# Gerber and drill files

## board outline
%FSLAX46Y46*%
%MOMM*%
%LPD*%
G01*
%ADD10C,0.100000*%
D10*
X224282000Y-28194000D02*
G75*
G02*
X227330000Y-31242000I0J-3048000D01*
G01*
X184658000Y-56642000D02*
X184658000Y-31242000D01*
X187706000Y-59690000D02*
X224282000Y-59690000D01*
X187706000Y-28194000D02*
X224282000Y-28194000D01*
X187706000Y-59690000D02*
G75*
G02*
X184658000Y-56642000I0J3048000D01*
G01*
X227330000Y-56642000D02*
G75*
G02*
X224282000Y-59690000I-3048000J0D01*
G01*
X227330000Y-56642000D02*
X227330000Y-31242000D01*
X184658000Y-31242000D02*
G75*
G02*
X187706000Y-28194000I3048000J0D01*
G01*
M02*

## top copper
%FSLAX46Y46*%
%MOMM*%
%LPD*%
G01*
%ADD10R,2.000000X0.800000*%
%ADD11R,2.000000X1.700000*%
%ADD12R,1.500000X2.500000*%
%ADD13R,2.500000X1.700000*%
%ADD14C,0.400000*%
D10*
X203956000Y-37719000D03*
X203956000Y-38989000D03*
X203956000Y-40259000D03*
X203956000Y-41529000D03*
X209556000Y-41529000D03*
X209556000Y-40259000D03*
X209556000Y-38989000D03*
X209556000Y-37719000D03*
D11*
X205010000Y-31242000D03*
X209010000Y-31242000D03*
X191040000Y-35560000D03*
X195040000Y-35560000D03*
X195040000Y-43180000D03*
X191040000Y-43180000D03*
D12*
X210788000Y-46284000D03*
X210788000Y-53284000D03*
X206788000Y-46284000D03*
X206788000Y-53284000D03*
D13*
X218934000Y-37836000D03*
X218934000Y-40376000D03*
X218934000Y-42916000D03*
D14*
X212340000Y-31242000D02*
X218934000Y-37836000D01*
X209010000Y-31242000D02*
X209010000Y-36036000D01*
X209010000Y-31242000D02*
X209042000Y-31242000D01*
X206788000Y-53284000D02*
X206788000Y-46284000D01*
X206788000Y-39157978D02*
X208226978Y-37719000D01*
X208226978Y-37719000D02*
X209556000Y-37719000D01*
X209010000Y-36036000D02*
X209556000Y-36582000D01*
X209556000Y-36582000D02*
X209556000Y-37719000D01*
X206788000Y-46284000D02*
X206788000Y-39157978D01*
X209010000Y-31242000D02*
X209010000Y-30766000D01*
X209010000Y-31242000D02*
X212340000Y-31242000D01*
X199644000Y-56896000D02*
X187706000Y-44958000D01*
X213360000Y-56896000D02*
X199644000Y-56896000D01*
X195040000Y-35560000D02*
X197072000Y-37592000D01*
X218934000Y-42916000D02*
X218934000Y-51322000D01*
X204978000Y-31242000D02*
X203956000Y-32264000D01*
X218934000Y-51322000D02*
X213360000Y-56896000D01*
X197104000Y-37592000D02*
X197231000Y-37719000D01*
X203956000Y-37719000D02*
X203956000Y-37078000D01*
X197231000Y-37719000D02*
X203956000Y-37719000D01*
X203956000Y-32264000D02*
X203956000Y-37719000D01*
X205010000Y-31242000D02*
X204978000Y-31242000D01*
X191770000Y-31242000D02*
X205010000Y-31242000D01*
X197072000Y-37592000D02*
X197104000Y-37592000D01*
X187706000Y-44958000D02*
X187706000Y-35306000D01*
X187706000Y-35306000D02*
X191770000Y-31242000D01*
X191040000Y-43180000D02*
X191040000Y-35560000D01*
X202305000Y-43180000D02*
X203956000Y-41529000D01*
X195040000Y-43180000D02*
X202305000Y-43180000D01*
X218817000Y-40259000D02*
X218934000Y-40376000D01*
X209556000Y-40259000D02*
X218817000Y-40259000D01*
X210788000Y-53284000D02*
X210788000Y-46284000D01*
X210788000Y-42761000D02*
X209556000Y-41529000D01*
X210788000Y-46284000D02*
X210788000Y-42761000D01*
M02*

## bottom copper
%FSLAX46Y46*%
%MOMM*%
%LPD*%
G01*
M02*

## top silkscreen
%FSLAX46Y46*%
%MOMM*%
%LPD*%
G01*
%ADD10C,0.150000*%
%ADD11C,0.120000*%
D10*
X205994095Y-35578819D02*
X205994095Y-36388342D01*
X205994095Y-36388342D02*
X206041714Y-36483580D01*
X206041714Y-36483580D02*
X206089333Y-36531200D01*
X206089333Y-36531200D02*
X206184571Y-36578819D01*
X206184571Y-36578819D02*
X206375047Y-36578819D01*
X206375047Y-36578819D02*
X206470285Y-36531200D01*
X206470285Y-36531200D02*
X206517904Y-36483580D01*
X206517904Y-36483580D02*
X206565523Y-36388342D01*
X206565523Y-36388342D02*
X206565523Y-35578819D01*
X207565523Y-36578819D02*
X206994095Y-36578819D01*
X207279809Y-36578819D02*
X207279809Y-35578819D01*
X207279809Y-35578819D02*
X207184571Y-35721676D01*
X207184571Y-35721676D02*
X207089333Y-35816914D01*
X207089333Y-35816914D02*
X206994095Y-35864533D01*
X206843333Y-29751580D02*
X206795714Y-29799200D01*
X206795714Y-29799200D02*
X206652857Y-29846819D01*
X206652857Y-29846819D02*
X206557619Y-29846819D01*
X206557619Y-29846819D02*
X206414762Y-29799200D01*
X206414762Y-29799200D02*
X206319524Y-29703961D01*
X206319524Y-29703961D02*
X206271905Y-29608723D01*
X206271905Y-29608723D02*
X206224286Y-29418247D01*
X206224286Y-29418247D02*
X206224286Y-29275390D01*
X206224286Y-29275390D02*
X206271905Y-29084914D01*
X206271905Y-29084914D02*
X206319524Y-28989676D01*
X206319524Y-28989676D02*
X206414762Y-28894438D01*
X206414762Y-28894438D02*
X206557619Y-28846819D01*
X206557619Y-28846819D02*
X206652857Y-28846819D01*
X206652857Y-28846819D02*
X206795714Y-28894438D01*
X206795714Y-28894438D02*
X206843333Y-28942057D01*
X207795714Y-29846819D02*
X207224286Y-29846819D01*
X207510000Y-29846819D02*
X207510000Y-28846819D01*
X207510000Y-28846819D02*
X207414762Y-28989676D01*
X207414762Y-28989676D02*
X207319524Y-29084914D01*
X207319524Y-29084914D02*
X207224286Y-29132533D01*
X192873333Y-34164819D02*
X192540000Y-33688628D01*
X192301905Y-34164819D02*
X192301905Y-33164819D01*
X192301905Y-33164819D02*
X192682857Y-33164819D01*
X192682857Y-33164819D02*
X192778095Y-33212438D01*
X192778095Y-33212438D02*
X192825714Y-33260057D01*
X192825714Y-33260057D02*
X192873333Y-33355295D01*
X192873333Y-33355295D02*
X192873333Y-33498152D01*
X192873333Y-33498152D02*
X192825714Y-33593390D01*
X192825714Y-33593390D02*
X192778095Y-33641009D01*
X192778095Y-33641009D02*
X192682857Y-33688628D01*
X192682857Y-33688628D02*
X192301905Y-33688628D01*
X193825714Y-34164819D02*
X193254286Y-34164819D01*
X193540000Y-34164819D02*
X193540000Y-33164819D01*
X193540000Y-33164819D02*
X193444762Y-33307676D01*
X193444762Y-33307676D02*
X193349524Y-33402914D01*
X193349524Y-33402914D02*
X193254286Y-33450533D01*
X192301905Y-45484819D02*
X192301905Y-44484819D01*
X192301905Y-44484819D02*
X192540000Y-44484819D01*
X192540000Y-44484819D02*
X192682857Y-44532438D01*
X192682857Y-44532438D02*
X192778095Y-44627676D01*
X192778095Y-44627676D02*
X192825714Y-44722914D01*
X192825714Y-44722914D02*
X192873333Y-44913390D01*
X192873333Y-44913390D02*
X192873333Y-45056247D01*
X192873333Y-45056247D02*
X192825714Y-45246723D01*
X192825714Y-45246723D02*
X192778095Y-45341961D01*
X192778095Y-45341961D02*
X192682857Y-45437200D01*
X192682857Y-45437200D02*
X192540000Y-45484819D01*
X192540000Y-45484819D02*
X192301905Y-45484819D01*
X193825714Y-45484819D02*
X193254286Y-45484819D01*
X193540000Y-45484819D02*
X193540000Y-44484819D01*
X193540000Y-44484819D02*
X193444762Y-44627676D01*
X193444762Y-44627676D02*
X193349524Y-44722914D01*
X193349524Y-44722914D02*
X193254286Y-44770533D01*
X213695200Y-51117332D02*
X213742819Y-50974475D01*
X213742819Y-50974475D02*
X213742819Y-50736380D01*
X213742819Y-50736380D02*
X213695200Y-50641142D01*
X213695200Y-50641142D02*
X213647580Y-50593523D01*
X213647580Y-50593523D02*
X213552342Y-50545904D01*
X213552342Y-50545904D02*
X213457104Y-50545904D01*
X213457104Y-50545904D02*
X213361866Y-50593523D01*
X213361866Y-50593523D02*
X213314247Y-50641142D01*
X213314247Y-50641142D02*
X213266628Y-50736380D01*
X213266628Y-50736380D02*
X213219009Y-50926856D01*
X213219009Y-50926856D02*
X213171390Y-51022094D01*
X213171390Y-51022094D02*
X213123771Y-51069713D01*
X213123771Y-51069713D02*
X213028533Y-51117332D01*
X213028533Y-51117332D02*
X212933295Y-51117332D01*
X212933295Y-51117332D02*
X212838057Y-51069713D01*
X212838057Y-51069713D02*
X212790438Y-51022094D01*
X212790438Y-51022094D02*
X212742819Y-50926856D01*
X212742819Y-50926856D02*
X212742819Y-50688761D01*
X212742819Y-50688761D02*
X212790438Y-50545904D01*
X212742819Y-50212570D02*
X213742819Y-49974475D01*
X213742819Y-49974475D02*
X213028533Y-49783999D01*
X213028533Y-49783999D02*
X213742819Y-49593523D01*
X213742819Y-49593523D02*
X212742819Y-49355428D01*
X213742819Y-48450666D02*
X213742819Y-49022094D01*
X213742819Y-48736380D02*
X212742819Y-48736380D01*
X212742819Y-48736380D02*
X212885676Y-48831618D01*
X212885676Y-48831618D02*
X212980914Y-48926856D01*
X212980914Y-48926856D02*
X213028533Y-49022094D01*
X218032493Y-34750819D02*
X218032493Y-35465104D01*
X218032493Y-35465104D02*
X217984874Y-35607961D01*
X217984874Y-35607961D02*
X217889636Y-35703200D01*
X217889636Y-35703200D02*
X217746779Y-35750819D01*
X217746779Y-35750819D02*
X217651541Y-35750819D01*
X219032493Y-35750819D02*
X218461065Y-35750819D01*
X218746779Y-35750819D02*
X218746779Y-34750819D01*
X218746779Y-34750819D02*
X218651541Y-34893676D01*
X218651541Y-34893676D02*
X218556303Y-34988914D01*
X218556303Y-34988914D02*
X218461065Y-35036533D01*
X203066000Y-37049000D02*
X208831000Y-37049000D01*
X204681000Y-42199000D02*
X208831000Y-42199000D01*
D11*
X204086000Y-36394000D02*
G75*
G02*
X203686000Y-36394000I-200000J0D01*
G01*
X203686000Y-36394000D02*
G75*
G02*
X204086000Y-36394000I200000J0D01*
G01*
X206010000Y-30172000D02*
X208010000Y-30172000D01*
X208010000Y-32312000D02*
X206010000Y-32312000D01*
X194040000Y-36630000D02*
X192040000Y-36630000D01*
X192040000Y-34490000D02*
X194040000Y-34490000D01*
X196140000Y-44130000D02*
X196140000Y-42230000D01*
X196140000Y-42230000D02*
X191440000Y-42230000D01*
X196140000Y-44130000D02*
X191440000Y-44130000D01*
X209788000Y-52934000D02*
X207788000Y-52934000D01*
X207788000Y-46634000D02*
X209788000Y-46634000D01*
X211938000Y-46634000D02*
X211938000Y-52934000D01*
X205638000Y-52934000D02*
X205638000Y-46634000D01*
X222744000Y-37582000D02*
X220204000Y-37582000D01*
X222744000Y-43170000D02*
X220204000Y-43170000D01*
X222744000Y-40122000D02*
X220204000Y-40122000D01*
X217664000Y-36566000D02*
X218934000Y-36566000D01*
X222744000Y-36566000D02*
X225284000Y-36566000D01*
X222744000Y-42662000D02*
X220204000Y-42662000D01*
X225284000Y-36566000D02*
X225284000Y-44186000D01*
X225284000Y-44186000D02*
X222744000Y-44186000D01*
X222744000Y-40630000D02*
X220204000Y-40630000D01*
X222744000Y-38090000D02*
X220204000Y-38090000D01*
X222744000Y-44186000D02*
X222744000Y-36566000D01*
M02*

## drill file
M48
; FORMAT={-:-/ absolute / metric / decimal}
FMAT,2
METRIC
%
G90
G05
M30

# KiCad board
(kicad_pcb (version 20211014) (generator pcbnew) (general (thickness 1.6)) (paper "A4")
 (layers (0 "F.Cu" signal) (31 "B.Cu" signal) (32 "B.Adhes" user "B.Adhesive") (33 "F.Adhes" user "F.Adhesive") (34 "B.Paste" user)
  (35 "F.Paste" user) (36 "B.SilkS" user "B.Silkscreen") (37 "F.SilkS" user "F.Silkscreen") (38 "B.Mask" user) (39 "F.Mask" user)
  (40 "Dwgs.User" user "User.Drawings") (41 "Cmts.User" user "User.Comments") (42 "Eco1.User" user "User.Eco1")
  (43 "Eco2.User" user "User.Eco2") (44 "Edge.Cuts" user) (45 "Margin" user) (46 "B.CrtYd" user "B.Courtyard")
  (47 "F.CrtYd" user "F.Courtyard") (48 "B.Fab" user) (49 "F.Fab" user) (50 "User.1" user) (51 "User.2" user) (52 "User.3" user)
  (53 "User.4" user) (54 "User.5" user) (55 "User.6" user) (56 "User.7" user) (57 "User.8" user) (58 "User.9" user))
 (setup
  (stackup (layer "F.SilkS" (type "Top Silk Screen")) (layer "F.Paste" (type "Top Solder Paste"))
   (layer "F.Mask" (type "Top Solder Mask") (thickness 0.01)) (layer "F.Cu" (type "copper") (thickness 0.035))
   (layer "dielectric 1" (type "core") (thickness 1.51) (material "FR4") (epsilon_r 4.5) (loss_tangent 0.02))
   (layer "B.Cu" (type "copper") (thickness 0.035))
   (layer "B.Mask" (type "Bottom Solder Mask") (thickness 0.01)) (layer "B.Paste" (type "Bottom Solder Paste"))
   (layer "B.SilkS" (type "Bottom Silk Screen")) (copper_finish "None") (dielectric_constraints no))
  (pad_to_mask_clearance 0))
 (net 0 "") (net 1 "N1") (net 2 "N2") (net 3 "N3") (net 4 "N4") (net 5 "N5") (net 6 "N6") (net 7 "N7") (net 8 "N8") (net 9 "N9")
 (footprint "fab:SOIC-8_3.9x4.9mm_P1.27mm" (layer "F.Cu") (at 206.756 39.624)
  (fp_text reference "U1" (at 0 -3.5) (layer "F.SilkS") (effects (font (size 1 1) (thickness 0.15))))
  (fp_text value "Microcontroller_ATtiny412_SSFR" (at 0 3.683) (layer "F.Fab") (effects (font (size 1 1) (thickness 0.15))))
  (fp_line (start -3.69 -2.575) (end 2.075 -2.575) (layer "F.SilkS") (width 0.15))
  (fp_line (start -2.075 2.575) (end 2.075 2.575) (layer "F.SilkS") (width 0.15))
  (fp_circle (center -2.87 -3.23) (end -2.67 -3.23) (layer "F.SilkS") (width 0.12) (fill none))
  (pad "1" smd rect locked (at -2.8 -1.905) (size 2 0.8) (layers "F.Cu" "F.Paste" "F.Mask") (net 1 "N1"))
  (pad "2" smd rect locked (at -2.8 -0.635) (size 2 0.8) (layers "F.Cu" "F.Paste" "F.Mask") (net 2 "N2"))
  (pad "3" smd rect locked (at -2.8 0.635) (size 2 0.8) (layers "F.Cu" "F.Paste" "F.Mask") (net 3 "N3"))
  (pad "4" smd rect locked (at -2.8 1.905) (size 2 0.8) (layers "F.Cu" "F.Paste" "F.Mask") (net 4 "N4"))
  (pad "5" smd rect locked (at 2.8 1.905) (size 2 0.8) (layers "F.Cu" "F.Paste" "F.Mask") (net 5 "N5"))
  (pad "6" smd rect locked (at 2.8 0.635) (size 2 0.8) (layers "F.Cu" "F.Paste" "F.Mask") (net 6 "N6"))
  (pad "7" smd rect locked (at 2.8 -0.635) (size 2 0.8) (layers "F.Cu" "F.Paste" "F.Mask") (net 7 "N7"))
  (pad "8" smd rect locked (at 2.8 -1.905) (size 2 0.8) (layers "F.Cu" "F.Paste" "F.Mask") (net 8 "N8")))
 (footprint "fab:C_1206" (layer "F.Cu") (at 207.01 31.242)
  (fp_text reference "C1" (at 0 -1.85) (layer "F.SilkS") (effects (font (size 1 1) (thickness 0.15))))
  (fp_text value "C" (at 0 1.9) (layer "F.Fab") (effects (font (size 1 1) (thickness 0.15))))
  (fp_line (start -1 -1.07) (end 1 -1.07) (layer "F.SilkS") (width 0.12))
  (fp_line (start 1 1.07) (end -1 1.07) (layer "F.SilkS") (width 0.12))
  (pad "1" smd rect locked (at -2 0) (size 2 1.7) (layers "F.Cu" "F.Paste" "F.Mask") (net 1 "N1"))
  (pad "2" smd rect locked (at 2 0) (size 2 1.7) (layers "F.Cu" "F.Paste" "F.Mask") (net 8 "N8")))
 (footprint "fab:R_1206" (layer "F.Cu") (at 193.04 35.56)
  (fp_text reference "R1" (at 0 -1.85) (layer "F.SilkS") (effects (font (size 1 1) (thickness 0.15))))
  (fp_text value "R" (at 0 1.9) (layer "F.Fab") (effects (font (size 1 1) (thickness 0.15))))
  (fp_line (start 1 1.07) (end -1 1.07) (layer "F.SilkS") (width 0.12))
  (fp_line (start -1 -1.07) (end 1 -1.07) (layer "F.SilkS") (width 0.12))
  (pad "1" smd rect locked (at -2 0) (size 2 1.7) (layers "F.Cu" "F.Paste" "F.Mask") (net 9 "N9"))
  (pad "2" smd rect locked (at 2 0) (size 2 1.7) (layers "F.Cu" "F.Paste" "F.Mask") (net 1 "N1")))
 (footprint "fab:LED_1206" (layer "F.Cu") (at 193.04 43.18 180)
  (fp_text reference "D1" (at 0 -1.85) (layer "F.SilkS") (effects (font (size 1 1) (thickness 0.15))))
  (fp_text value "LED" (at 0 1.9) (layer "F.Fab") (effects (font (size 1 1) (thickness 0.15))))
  (fp_line (start -3.1 -0.95) (end -3.1 0.95) (layer "F.SilkS") (width 0.12))
  (fp_line (start -3.1 0.95) (end 1.6 0.95) (layer "F.SilkS") (width 0.12))
  (fp_line (start -3.1 -0.95) (end 1.6 -0.95) (layer "F.SilkS") (width 0.12))
  (pad "1" smd rect locked (at -2 0 180) (size 2 1.7) (layers "F.Cu" "F.Paste" "F.Mask") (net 4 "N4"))
  (pad "2" smd rect locked (at 2 0 180) (size 2 1.7) (layers "F.Cu" "F.Paste" "F.Mask") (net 9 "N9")))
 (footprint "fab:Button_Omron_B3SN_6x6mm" (layer "F.Cu") (at 208.788 49.784 -90)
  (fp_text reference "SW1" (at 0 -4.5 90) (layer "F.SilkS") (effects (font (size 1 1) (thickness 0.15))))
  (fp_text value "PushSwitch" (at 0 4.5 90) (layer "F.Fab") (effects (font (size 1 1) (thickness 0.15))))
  (fp_line (start 3.15 -1) (end 3.15 1) (layer "F.SilkS") (width 0.12))
  (fp_line (start -3.15 1) (end -3.15 -1) (layer "F.SilkS") (width 0.12))
  (fp_line (start -3.15 -3.15) (end 3.15 -3.15) (layer "F.SilkS") (width 0.12))
  (fp_line (start 3.15 3.15) (end -3.15 3.15) (layer "F.SilkS") (width 0.12))
  (pad "1" smd rect locked (at -3.5 -2 270) (size 2.5 1.5) (layers "F.Cu" "F.Paste" "F.Mask") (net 5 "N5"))
  (pad "1" smd rect locked (at 3.5 -2 270) (size 2.5 1.5) (layers "F.Cu" "F.Paste" "F.Mask") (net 5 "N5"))
  (pad "2" smd rect locked (at -3.5 2 270) (size 2.5 1.5) (layers "F.Cu" "F.Paste" "F.Mask") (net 8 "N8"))
  (pad "2" smd rect locked (at 3.5 2 270) (size 2.5 1.5) (layers "F.Cu" "F.Paste" "F.Mask") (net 8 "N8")))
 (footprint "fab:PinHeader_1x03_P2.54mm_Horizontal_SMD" (layer "F.Cu") (at 218.934 37.836)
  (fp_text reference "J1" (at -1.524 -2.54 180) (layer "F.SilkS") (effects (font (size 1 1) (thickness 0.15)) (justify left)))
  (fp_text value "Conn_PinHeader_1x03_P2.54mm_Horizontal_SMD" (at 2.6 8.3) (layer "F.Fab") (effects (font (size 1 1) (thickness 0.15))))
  (fp_line (start 3.81 -0.254) (end 1.27 -0.254) (layer "F.SilkS") (width 0.12))
  (fp_line (start 3.81 5.334) (end 1.27 5.334) (layer "F.SilkS") (width 0.12))
  (fp_line (start 3.81 2.286) (end 1.27 2.286) (layer "F.SilkS") (width 0.12))
  (fp_line (start -1.27 -1.27) (end 0 -1.27) (layer "F.SilkS") (width 0.12))
  (fp_line (start 3.81 -1.27) (end 6.35 -1.27) (layer "F.SilkS") (width 0.12))
  (fp_line (start 3.81 4.826) (end 1.27 4.826) (layer "F.SilkS") (width 0.12))
  (fp_line (start 6.35 -1.27) (end 6.35 6.35) (layer "F.SilkS") (width 0.12))
  (fp_line (start 6.35 6.35) (end 3.81 6.35) (layer "F.SilkS") (width 0.12))
  (fp_line (start 3.81 2.794) (end 1.27 2.794) (layer "F.SilkS") (width 0.12))
  (fp_line (start 3.81 0.254) (end 1.27 0.254) (layer "F.SilkS") (width 0.12))
  (fp_line (start 3.81 6.35) (end 3.81 -1.27) (layer "F.SilkS") (width 0.12))
  (pad "1" smd rect locked (at 0 0) (size 2.5 1.7) (layers "F.Cu" "F.Paste" "F.Mask") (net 8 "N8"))
  (pad "2" smd rect locked (at 0 2.54) (size 2.5 1.7) (layers "F.Cu" "F.Paste" "F.Mask") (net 6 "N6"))
  (pad "3" smd rect locked (at 0 5.08) (size 2.5 1.7) (layers "F.Cu" "F.Paste" "F.Mask") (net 1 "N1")))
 (gr_arc (start 224.282 28.194) (mid 226.437261 29.086739) (end 227.33 31.242) (layer "Edge.Cuts") (width 0.1))
 (gr_line (start 184.658 56.642) (end 184.658 31.242) (layer "Edge.Cuts") (width 0.1))
 (gr_line (start 187.706 59.69) (end 224.282 59.69) (layer "Edge.Cuts") (width 0.1))
 (gr_line (start 187.706 28.194) (end 224.282 28.194) (layer "Edge.Cuts") (width 0.1))
 (gr_arc (start 187.706 59.69) (mid 185.550739 58.797261) (end 184.658 56.642) (layer "Edge.Cuts") (width 0.1))
 (gr_arc (start 227.33 56.642) (mid 226.437261 58.797261) (end 224.282 59.69) (layer "Edge.Cuts") (width 0.1))
 (gr_line (start 227.33 56.642) (end 227.33 31.242) (layer "Edge.Cuts") (width 0.1))
 (gr_arc (start 184.658 31.242) (mid 185.550739 29.086739) (end 187.706 28.194) (layer "Edge.Cuts") (width 0.1))
 (segment (start 212.34 31.242) (end 218.934 37.836) (width 0.4) (layer "F.Cu") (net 8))
 (segment (start 209.01 31.242) (end 209.01 36.036) (width 0.4) (layer "F.Cu") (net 8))
 (segment (start 209.01 31.242) (end 209.042 31.242) (width 0.4) (layer "F.Cu") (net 8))
 (segment (start 206.788 53.284) (end 206.788 46.284) (width 0.4) (layer "F.Cu") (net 8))
 (segment (start 206.788 39.157978) (end 208.226978 37.719) (width 0.4) (layer "F.Cu") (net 8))
 (segment (start 208.226978 37.719) (end 209.556 37.719) (width 0.4) (layer "F.Cu") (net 8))
 (segment (start 209.01 36.036) (end 209.556 36.582) (width 0.4) (layer "F.Cu") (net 8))
 (segment (start 209.556 36.582) (end 209.556 37.719) (width 0.4) (layer "F.Cu") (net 8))
 (segment (start 206.788 46.284) (end 206.788 39.157978) (width 0.4) (layer "F.Cu") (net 8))
 (segment (start 209.01 31.242) (end 209.01 30.766) (width 0.4) (layer "F.Cu") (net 8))
 (segment (start 209.01 31.242) (end 212.34 31.242) (width 0.4) (layer "F.Cu") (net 8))
 (segment (start 199.644 56.896) (end 187.706 44.958) (width 0.4) (layer "F.Cu") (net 1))
 (segment (start 213.36 56.896) (end 199.644 56.896) (width 0.4) (layer "F.Cu") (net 1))
 (segment (start 195.04 35.56) (end 197.072 37.592) (width 0.4) (layer "F.Cu") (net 1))
 (segment (start 218.934 42.916) (end 218.934 51.322) (width 0.4) (layer "F.Cu") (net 1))
 (segment (start 204.978 31.242) (end 203.956 32.264) (width 0.4) (layer "F.Cu") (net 1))
 (segment (start 218.934 51.322) (end 213.36 56.896) (width 0.4) (layer "F.Cu") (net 1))
 (segment (start 197.104 37.592) (end 197.231 37.719) (width 0.4) (layer "F.Cu") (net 1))
 (segment (start 203.956 37.719) (end 203.956 37.078) (width 0.4) (layer "F.Cu") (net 1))
 (segment (start 197.231 37.719) (end 203.956 37.719) (width 0.4) (layer "F.Cu") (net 1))
 (segment (start 203.956 32.264) (end 203.956 37.719) (width 0.4) (layer "F.Cu") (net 1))
 (segment (start 205.01 31.242) (end 204.978 31.242) (width 0.4) (layer "F.Cu") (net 1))
 (segment (start 191.77 31.242) (end 205.01 31.242) (width 0.4) (layer "F.Cu") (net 1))
 (segment (start 197.072 37.592) (end 197.104 37.592) (width 0.4) (layer "F.Cu") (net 1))
 (segment (start 187.706 44.958) (end 187.706 35.306) (width 0.4) (layer "F.Cu") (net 1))
 (segment (start 187.706 35.306) (end 191.77 31.242) (width 0.4) (layer "F.Cu") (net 1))
 (segment (start 191.04 43.18) (end 191.04 35.56) (width 0.4) (layer "F.Cu") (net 9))
 (segment (start 202.305 43.18) (end 203.956 41.529) (width 0.4) (layer "F.Cu") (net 4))
 (segment (start 195.04 43.18) (end 202.305 43.18) (width 0.4) (layer "F.Cu") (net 4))
 (segment (start 218.817 40.259) (end 218.934 40.376) (width 0.4) (layer "F.Cu") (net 6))
 (segment (start 209.556 40.259) (end 218.817 40.259) (width 0.4) (layer "F.Cu") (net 6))
 (segment (start 210.788 53.284) (end 210.788 46.284) (width 0.4) (layer "F.Cu") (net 5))
 (segment (start 210.788 42.761) (end 209.556 41.529) (width 0.4) (layer "F.Cu") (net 5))
 (segment (start 210.788 46.284) (end 210.788 42.761) (width 0.4) (layer "F.Cu") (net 5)))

